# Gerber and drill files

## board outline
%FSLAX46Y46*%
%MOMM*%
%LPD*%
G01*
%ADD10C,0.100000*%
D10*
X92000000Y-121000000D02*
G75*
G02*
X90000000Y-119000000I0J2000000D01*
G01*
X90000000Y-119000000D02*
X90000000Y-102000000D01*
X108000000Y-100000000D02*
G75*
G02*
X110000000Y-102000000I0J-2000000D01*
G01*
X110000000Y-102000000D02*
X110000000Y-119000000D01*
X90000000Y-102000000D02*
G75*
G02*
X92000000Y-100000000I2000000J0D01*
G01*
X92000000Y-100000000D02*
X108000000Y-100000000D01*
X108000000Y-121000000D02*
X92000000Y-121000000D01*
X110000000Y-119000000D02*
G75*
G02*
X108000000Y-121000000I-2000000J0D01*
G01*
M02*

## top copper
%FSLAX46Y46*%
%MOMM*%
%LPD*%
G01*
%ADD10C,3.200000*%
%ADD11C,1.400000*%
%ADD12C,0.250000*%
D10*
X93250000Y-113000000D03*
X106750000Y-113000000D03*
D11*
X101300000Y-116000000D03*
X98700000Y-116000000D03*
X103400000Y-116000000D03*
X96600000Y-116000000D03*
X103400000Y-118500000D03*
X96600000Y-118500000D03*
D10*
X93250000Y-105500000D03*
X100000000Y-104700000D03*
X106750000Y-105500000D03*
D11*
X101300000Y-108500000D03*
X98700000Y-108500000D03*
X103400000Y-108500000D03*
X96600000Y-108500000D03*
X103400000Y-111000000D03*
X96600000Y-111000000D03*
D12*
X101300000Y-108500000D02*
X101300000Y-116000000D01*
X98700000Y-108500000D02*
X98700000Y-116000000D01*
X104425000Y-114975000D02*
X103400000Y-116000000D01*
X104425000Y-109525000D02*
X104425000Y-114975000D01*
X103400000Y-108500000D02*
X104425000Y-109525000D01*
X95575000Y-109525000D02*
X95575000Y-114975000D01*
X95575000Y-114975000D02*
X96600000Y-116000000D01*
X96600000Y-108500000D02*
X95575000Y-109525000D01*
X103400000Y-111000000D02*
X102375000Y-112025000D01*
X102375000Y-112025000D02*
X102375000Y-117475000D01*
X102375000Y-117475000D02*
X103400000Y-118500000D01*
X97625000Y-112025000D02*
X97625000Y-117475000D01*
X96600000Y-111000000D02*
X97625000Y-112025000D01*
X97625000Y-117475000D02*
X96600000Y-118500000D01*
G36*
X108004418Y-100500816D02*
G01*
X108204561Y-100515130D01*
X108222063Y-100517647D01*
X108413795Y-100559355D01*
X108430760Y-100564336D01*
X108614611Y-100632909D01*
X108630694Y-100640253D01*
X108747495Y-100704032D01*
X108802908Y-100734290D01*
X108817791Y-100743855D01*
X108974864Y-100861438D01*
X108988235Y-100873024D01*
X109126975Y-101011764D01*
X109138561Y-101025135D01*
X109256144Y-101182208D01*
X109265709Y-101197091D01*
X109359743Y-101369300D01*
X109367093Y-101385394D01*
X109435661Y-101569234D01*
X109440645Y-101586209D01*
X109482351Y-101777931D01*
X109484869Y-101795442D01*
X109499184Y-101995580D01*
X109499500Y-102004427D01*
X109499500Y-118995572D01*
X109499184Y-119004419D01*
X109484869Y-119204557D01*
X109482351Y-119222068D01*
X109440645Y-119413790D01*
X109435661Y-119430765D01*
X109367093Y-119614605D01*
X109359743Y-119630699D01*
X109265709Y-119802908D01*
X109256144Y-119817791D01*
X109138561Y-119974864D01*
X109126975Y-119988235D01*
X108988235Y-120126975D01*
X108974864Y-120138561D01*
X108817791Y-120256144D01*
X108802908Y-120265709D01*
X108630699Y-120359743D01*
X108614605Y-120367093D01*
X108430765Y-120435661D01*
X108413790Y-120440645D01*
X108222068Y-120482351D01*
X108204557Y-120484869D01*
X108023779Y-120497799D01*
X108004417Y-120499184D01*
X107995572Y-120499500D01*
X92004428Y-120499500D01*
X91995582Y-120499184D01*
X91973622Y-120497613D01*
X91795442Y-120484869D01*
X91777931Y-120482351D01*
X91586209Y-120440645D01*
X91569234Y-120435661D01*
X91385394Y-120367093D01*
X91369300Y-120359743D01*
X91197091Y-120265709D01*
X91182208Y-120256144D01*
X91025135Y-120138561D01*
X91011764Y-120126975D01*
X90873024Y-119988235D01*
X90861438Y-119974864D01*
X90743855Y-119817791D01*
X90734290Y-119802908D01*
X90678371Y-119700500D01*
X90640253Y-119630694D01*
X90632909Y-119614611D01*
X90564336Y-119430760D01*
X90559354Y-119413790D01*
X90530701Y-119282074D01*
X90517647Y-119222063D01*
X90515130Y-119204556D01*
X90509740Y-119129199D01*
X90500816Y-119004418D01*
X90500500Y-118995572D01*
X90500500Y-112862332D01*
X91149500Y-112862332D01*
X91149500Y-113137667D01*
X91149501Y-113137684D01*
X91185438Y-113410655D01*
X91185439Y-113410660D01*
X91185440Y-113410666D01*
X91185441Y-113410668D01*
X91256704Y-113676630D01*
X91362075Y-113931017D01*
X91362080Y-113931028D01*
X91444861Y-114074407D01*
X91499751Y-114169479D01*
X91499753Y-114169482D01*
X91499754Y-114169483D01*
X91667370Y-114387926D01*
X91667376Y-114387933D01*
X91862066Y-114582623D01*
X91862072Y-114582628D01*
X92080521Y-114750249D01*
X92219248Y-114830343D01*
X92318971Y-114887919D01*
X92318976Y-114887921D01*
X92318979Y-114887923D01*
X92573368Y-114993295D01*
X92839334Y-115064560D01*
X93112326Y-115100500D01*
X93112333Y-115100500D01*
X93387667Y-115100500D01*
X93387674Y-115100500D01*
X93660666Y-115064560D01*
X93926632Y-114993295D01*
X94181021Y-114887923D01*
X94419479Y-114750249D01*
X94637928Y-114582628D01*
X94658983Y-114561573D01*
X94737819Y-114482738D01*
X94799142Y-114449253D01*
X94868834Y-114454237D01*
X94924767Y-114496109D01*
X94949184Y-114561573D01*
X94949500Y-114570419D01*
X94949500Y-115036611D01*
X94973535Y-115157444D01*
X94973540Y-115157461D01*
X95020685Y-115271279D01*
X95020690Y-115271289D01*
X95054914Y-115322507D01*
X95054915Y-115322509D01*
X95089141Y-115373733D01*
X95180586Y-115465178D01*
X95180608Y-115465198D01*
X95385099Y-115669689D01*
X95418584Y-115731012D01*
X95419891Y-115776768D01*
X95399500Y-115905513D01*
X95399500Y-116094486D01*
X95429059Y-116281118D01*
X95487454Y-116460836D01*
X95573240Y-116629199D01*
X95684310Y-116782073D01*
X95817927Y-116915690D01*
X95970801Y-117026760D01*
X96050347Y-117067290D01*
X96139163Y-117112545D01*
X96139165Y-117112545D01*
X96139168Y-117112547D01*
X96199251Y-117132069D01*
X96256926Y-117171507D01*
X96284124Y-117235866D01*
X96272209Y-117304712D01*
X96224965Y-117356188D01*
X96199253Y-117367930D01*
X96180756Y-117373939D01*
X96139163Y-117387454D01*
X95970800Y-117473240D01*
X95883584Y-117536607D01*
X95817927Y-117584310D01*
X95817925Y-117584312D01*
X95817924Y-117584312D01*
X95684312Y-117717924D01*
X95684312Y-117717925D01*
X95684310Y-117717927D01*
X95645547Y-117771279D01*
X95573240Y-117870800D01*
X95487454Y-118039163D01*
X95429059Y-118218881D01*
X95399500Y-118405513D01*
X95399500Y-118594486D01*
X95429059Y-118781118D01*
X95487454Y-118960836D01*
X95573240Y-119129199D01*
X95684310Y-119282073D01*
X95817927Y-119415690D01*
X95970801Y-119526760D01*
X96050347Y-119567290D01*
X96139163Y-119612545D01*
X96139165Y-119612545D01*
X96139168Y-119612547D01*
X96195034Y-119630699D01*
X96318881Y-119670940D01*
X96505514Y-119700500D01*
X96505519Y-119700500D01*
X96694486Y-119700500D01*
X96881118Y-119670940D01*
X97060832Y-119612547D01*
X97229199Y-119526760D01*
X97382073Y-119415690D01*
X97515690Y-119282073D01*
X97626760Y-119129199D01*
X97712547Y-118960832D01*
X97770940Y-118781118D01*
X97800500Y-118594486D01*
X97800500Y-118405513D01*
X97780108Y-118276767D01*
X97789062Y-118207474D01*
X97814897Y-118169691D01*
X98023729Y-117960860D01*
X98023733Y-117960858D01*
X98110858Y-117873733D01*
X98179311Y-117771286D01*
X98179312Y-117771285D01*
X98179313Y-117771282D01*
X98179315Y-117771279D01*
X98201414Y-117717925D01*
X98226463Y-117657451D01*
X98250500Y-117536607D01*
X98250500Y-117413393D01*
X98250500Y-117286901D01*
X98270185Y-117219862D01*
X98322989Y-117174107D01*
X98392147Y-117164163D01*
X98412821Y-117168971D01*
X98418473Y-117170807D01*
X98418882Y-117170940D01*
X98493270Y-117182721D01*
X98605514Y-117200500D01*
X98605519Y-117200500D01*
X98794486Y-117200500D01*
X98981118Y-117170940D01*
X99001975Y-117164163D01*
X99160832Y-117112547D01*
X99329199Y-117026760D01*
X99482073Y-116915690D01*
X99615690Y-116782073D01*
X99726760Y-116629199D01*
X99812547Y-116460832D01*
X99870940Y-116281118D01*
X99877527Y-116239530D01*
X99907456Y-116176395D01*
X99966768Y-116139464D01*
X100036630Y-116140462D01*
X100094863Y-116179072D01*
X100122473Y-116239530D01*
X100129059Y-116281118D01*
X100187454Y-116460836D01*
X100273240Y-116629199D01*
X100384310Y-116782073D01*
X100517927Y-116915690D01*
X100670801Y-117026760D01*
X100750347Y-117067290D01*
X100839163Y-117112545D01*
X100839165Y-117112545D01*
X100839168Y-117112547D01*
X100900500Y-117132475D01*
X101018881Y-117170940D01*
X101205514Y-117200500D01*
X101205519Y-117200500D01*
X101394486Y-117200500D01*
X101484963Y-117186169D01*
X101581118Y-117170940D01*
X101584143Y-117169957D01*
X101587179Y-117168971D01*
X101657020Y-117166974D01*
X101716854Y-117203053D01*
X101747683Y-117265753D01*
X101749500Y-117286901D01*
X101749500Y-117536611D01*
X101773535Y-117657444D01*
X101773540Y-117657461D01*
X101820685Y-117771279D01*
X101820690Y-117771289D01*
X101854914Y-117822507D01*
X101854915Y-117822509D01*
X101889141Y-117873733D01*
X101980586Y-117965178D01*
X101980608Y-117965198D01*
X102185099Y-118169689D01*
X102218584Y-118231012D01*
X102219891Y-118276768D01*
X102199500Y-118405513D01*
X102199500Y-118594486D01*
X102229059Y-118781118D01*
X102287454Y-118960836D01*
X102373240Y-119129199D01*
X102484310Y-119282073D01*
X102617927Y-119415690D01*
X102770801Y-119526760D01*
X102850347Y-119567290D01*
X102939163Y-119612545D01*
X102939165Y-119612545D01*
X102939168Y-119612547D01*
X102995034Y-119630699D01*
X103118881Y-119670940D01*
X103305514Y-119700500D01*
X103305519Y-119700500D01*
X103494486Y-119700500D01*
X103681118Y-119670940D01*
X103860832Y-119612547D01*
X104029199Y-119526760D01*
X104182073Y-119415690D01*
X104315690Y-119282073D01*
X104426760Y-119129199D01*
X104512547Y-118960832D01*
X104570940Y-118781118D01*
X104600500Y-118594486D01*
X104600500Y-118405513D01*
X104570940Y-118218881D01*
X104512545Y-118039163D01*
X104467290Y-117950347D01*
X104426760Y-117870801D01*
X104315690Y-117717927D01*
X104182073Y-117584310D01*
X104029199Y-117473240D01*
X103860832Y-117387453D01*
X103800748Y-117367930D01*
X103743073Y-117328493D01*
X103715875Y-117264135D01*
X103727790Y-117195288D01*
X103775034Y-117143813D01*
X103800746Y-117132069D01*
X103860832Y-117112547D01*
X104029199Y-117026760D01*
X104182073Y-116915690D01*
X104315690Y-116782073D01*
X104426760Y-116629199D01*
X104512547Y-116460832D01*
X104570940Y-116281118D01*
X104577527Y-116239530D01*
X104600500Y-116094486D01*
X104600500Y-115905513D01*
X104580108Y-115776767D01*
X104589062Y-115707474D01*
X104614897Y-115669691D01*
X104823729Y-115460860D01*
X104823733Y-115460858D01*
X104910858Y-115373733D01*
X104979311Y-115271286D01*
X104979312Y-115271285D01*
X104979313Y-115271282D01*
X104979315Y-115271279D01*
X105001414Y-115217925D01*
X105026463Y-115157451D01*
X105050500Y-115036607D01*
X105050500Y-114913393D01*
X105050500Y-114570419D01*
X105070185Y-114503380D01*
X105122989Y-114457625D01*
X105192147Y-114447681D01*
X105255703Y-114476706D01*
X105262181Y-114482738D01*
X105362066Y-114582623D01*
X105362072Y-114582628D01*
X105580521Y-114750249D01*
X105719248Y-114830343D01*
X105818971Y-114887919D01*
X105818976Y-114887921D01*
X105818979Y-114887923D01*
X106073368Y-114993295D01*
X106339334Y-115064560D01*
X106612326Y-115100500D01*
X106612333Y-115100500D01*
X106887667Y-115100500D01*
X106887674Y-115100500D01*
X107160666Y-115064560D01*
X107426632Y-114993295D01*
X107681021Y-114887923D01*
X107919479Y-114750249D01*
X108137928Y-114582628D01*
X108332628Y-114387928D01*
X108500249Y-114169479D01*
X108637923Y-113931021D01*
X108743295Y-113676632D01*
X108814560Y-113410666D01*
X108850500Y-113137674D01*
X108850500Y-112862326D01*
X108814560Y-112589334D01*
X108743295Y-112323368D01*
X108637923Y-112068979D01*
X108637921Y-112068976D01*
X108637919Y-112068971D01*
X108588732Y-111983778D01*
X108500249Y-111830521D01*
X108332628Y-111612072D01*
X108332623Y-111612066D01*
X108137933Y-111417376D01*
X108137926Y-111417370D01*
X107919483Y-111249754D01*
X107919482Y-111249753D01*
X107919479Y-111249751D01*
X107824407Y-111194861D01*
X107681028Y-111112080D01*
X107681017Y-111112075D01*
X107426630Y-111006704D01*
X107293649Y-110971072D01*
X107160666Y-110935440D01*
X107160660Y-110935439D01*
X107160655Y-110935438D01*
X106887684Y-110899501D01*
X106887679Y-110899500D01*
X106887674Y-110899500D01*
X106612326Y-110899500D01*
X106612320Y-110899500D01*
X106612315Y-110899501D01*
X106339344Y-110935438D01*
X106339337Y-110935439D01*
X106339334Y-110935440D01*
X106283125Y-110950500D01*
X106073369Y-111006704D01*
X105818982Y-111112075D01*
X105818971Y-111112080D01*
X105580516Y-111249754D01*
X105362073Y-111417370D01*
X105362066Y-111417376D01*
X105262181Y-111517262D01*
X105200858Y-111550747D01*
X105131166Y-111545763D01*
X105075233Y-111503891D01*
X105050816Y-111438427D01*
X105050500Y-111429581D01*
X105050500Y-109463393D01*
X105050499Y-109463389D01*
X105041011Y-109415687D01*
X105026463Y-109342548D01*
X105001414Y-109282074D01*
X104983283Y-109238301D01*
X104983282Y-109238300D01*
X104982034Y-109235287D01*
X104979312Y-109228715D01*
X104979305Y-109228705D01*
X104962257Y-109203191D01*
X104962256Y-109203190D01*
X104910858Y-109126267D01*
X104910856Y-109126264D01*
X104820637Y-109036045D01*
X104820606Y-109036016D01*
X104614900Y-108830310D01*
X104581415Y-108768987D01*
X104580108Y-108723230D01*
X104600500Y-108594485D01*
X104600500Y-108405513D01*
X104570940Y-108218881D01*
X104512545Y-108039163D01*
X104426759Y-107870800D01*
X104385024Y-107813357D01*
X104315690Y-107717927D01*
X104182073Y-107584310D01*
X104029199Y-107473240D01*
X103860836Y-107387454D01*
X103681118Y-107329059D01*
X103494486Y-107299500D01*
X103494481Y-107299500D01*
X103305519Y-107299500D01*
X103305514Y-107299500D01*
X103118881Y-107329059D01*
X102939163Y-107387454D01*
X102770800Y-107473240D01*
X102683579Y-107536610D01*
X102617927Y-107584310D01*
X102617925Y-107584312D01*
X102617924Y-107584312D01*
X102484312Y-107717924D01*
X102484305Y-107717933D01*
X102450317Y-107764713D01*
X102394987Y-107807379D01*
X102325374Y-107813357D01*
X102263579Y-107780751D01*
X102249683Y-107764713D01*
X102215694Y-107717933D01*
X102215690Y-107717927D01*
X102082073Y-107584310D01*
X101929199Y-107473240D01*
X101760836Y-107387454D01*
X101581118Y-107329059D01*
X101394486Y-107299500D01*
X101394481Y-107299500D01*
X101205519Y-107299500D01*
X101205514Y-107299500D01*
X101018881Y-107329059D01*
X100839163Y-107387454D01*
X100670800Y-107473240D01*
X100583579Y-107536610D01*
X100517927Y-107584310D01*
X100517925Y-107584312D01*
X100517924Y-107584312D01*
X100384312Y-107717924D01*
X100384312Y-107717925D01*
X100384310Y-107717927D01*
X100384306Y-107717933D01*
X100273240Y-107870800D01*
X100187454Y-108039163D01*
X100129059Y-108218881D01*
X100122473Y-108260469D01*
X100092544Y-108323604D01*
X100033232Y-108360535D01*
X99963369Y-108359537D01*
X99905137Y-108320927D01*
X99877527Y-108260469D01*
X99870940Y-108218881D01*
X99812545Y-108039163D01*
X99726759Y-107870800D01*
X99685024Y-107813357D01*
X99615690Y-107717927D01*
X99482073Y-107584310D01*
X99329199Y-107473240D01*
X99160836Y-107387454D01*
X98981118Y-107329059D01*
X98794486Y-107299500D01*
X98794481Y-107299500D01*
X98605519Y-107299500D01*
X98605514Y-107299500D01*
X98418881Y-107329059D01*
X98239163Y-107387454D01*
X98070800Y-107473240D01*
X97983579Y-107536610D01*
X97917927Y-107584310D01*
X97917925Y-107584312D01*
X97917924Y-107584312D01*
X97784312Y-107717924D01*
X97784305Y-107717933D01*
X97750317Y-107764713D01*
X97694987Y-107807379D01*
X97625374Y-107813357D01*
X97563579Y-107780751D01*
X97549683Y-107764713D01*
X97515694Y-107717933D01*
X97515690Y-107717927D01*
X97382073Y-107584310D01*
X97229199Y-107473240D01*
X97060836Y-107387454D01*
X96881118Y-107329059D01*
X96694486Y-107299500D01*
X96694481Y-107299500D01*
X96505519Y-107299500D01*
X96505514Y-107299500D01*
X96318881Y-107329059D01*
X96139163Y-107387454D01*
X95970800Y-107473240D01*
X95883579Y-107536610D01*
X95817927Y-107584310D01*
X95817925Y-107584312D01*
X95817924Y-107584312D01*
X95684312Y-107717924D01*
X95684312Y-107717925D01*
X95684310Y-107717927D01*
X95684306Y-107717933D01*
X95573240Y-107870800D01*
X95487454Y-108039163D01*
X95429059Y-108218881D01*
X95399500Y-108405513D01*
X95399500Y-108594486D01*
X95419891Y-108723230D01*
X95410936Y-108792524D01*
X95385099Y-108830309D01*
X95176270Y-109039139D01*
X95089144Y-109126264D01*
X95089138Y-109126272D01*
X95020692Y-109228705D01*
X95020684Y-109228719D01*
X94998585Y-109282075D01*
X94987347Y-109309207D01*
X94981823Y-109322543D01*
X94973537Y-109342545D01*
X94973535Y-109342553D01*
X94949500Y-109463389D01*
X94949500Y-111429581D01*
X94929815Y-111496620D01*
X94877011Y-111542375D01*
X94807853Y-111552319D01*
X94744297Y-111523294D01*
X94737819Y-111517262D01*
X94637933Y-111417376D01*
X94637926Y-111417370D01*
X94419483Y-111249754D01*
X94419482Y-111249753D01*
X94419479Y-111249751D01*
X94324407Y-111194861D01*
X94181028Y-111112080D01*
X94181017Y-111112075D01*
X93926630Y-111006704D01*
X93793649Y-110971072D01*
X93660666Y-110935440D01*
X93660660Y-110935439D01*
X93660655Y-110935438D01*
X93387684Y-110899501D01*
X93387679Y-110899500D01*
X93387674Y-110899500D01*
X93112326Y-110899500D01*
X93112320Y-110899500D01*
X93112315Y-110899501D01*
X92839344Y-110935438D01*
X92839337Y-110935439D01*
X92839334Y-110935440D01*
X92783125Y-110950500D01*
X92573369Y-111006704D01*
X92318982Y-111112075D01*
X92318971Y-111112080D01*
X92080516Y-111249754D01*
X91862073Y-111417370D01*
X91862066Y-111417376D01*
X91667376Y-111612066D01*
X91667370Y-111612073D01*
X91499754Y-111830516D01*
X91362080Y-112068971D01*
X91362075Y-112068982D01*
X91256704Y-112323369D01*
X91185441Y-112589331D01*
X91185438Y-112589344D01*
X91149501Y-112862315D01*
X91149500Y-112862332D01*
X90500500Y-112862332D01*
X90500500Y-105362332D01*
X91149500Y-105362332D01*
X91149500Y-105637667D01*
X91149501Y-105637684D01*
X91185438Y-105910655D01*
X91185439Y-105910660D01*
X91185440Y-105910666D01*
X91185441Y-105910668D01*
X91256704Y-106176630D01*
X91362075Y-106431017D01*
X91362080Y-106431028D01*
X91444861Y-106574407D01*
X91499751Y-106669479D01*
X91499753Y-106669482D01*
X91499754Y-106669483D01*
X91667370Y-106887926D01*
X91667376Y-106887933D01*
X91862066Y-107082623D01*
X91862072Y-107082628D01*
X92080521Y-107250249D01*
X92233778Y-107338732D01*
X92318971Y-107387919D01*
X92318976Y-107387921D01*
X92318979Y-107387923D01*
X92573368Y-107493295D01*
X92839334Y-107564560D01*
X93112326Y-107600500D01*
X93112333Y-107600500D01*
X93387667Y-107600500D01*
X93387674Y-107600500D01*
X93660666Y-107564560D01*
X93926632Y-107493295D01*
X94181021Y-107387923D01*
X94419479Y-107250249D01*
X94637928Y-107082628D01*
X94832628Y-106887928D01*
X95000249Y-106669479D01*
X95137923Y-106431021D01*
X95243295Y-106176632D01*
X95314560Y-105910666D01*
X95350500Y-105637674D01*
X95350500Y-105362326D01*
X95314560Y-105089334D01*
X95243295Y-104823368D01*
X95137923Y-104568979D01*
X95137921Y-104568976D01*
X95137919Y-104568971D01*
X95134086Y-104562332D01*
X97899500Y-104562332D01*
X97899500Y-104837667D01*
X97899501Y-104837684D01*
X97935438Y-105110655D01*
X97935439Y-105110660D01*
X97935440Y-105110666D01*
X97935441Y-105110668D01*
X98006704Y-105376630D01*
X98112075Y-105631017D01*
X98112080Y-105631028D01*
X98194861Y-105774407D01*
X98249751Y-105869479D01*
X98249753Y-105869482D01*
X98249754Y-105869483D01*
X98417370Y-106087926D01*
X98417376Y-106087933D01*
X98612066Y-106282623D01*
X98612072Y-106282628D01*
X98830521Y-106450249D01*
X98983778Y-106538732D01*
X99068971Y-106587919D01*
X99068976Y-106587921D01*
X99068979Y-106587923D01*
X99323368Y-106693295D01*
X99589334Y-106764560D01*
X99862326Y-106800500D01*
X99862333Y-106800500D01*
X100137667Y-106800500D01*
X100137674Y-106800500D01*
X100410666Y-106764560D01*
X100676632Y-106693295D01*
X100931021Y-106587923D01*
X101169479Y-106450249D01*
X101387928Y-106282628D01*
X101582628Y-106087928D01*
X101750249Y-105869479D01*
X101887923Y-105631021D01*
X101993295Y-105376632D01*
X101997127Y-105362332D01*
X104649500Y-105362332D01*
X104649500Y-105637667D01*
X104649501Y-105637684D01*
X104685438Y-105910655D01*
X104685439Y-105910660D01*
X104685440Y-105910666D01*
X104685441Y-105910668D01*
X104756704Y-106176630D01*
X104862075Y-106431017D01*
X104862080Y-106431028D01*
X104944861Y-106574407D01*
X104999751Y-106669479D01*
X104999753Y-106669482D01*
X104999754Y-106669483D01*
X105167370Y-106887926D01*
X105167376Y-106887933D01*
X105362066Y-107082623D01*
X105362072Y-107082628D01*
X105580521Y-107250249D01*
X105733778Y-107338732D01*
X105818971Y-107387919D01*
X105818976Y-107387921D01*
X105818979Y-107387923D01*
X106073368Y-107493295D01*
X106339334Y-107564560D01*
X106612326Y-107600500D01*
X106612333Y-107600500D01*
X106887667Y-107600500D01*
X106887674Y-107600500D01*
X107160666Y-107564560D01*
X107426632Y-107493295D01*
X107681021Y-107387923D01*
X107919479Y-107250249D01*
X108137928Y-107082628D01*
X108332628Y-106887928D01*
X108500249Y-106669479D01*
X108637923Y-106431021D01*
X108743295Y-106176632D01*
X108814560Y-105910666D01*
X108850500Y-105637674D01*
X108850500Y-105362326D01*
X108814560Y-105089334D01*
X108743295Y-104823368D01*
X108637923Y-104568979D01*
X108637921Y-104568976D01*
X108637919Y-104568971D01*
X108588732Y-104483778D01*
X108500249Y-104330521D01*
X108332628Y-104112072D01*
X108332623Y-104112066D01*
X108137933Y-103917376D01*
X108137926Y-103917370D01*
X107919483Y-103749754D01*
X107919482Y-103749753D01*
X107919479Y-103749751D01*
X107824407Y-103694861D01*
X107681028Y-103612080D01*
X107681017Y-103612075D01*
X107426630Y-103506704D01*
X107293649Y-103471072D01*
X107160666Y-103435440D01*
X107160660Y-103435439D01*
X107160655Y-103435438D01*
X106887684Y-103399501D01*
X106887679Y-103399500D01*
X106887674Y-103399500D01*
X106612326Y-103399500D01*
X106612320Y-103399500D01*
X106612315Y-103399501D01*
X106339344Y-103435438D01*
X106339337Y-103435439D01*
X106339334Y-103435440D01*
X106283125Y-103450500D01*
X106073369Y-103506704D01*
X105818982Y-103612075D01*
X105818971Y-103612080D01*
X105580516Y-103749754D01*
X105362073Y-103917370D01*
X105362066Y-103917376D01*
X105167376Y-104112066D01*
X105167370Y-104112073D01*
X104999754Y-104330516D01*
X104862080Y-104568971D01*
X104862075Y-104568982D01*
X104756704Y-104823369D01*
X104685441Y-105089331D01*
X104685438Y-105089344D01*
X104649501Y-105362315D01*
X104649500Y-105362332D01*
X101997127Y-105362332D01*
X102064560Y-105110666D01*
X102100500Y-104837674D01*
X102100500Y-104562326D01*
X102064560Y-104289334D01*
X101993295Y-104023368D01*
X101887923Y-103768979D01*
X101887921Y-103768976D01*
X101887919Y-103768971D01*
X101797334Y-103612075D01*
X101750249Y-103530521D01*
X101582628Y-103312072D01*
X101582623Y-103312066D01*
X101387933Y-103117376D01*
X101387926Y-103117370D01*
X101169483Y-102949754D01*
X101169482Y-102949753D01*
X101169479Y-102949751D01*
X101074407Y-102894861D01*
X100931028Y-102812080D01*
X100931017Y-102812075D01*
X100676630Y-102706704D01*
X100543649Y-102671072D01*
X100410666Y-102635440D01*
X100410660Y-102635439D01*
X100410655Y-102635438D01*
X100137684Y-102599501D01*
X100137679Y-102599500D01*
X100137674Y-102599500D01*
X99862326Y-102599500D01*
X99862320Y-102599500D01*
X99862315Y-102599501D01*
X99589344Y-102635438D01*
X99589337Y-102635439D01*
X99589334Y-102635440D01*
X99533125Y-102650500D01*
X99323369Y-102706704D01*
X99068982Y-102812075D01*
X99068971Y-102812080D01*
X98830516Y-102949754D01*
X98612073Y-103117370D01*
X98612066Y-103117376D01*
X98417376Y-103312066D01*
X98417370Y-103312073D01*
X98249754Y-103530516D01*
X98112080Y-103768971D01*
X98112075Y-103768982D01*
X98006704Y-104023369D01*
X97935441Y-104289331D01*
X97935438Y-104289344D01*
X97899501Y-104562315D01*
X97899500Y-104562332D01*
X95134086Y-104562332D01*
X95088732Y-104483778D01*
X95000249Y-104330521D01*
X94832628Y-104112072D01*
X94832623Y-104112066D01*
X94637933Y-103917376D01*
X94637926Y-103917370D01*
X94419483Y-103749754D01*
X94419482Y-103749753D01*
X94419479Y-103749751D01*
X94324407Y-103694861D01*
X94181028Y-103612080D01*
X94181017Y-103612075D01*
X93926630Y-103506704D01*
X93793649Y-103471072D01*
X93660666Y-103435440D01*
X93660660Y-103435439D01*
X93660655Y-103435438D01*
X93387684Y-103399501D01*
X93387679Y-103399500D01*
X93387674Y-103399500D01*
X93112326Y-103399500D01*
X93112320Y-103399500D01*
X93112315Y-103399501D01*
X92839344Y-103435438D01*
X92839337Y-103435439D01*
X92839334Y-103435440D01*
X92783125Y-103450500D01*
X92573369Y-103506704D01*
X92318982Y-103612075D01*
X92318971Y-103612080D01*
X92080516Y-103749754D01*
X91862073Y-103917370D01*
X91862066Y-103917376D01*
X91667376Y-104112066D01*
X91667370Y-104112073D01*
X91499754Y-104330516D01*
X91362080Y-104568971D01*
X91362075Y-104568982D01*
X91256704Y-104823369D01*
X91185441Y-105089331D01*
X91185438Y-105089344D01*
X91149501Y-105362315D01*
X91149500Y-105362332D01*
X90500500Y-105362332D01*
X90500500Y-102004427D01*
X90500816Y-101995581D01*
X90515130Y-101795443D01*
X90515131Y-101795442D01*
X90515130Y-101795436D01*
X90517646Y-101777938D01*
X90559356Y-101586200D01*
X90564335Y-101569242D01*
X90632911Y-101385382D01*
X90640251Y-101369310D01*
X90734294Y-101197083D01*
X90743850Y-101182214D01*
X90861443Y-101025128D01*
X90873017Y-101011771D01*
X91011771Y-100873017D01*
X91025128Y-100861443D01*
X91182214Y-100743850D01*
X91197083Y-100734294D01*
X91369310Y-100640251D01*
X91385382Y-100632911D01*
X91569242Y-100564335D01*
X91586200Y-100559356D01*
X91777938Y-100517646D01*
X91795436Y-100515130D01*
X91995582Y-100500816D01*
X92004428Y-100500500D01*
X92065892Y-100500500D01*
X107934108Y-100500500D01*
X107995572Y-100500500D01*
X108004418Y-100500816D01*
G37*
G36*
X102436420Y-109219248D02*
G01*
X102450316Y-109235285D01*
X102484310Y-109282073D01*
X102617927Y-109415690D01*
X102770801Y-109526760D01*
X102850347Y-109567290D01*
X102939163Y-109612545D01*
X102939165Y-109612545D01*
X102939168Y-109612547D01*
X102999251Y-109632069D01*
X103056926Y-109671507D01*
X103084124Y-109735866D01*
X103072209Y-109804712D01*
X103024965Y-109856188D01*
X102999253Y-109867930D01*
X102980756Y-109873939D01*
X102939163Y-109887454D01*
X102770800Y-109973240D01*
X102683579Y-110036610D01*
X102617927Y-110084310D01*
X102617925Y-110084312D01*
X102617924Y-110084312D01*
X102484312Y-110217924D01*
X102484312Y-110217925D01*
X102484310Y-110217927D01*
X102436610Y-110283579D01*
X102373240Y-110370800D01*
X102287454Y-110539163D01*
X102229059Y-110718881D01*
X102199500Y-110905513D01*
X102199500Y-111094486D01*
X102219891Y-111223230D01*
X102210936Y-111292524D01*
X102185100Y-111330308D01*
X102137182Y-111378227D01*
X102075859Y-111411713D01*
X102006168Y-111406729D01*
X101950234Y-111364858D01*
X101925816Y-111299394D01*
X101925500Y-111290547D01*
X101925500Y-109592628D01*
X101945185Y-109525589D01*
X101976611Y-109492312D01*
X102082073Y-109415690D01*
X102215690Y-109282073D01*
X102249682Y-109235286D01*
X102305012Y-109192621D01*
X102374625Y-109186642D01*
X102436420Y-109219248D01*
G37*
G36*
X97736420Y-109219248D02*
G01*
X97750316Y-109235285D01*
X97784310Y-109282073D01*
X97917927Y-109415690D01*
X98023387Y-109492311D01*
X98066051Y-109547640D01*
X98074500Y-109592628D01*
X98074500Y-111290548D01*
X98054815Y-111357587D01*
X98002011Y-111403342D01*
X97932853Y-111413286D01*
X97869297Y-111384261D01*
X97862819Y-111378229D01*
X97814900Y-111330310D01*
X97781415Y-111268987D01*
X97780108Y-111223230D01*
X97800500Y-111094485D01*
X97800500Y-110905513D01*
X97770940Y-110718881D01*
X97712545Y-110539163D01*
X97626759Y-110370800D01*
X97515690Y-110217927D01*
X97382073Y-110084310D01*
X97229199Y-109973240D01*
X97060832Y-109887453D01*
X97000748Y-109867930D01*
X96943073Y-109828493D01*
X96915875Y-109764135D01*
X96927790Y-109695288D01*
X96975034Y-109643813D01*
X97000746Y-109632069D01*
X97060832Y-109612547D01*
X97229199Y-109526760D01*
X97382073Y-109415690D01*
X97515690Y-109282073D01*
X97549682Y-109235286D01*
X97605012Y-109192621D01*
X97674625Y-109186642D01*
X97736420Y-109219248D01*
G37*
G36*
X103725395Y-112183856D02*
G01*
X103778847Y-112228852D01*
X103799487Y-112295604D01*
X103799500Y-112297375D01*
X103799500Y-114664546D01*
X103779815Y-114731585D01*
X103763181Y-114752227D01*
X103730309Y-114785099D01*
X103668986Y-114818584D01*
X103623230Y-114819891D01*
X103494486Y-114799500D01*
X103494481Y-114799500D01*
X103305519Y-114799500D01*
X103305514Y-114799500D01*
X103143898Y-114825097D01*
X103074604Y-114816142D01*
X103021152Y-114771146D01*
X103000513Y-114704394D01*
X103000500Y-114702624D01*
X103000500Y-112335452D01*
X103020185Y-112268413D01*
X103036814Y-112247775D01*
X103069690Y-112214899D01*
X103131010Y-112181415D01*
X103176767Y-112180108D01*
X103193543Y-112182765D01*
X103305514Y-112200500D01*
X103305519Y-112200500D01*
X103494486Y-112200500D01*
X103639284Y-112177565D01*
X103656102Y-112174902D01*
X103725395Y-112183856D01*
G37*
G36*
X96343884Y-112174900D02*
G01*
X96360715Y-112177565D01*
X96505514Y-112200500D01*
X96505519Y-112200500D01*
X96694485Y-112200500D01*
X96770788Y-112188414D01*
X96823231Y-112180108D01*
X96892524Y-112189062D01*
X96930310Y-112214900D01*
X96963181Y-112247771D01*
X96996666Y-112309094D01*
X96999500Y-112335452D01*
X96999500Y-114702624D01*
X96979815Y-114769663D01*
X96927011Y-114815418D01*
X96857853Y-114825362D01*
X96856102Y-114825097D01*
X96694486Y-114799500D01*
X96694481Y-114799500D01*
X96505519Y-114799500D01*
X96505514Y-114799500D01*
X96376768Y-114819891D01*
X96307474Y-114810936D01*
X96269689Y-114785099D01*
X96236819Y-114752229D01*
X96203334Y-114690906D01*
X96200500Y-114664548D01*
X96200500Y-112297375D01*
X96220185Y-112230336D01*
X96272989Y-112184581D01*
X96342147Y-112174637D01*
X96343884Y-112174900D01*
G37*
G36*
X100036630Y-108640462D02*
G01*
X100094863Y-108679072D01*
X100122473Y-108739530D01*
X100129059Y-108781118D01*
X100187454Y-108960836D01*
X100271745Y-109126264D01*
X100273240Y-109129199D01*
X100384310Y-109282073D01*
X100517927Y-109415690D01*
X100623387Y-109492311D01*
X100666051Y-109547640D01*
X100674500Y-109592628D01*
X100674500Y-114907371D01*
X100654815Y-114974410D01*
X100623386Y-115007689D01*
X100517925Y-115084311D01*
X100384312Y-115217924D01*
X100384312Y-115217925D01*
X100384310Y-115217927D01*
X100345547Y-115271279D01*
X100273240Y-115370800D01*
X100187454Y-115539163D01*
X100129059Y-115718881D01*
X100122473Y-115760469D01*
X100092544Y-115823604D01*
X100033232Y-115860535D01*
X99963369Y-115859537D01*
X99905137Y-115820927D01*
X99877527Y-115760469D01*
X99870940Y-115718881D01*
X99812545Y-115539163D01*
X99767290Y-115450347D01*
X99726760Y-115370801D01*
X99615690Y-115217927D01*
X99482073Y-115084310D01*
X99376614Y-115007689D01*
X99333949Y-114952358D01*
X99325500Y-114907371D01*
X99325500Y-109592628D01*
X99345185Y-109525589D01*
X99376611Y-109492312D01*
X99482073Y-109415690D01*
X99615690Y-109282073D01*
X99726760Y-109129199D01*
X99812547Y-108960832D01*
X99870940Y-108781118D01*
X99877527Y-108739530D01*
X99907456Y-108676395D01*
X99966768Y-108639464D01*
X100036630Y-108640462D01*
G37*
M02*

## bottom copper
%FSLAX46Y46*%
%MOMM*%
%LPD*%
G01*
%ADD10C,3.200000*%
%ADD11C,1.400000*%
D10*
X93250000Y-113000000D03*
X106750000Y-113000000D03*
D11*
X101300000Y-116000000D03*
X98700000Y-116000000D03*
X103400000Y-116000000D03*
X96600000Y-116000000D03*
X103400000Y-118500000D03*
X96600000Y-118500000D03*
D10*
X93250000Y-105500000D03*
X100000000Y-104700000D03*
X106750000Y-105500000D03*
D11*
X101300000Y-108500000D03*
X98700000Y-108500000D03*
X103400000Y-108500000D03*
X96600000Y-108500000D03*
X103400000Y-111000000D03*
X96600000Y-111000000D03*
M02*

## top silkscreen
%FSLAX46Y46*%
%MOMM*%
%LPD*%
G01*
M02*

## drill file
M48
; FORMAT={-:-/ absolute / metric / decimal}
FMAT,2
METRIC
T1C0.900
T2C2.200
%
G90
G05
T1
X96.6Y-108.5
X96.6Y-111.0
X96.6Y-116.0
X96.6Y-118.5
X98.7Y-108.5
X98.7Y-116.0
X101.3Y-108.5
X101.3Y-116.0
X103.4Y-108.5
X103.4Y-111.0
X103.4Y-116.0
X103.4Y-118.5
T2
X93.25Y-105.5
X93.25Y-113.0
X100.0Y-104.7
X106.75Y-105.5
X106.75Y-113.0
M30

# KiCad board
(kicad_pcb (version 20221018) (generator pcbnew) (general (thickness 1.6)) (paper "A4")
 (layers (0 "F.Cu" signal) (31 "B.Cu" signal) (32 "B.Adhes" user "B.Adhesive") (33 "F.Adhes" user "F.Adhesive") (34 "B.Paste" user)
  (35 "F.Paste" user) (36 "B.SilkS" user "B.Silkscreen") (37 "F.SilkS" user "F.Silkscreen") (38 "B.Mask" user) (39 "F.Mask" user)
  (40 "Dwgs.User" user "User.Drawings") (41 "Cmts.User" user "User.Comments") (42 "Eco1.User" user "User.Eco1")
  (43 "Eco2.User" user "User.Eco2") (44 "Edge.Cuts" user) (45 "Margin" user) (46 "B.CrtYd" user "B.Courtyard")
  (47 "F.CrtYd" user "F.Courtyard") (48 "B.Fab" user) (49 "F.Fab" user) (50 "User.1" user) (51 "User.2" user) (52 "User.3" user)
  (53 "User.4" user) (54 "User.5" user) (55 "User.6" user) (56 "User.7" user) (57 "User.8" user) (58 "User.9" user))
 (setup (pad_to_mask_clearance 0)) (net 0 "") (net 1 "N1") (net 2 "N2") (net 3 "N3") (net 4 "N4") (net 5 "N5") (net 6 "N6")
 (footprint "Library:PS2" (layer "F.Cu") (at 100 107.5)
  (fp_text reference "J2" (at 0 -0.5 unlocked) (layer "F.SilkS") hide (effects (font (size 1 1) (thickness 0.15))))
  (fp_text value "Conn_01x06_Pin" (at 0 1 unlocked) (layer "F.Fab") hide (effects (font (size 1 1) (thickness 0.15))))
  (pad "" thru_hole circle (at -6.75 5.5) (size 3.2 3.2) (drill 2.2) (layers "*.Cu" "*.Mask"))
  (pad "" thru_hole circle (at 6.75 5.5 90) (size 3.2 3.2) (drill 2.2) (layers "*.Cu" "*.Mask"))
  (pad "1" thru_hole circle (at 1.3 8.5) (size 1.4 1.4) (drill 0.9) (layers "*.Cu" "*.Mask") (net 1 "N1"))
  (pad "2" thru_hole circle (at -1.3 8.5) (size 1.4 1.4) (drill 0.9) (layers "*.Cu" "*.Mask") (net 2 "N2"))
  (pad "3" thru_hole circle (at 3.4 8.5) (size 1.4 1.4) (drill 0.9) (layers "*.Cu" "*.Mask") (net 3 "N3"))
  (pad "4" thru_hole circle (at -3.4 8.5) (size 1.4 1.4) (drill 0.9) (layers "*.Cu" "*.Mask") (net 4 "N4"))
  (pad "5" thru_hole circle (at 3.4 11) (size 1.4 1.4) (drill 0.9) (layers "*.Cu" "*.Mask") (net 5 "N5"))
  (pad "6" thru_hole circle (at -3.4 11) (size 1.4 1.4) (drill 0.9) (layers "*.Cu" "*.Mask") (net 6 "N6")))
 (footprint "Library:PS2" (layer "F.Cu") (at 100 100)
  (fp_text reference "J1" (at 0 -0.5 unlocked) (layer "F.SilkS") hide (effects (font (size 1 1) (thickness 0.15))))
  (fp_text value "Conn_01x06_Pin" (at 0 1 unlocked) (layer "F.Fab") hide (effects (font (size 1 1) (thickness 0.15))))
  (pad "" thru_hole circle (at -6.75 5.5) (size 3.2 3.2) (drill 2.2) (layers "*.Cu" "*.Mask"))
  (pad "" thru_hole circle (at 0 4.7) (size 3.2 3.2) (drill 2.2) (layers "*.Cu" "*.Mask"))
  (pad "" thru_hole circle (at 6.75 5.5 90) (size 3.2 3.2) (drill 2.2) (layers "*.Cu" "*.Mask"))
  (pad "1" thru_hole circle (at 1.3 8.5) (size 1.4 1.4) (drill 0.9) (layers "*.Cu" "*.Mask") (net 1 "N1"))
  (pad "2" thru_hole circle (at -1.3 8.5) (size 1.4 1.4) (drill 0.9) (layers "*.Cu" "*.Mask") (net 2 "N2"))
  (pad "3" thru_hole circle (at 3.4 8.5) (size 1.4 1.4) (drill 0.9) (layers "*.Cu" "*.Mask") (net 3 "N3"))
  (pad "4" thru_hole circle (at -3.4 8.5) (size 1.4 1.4) (drill 0.9) (layers "*.Cu" "*.Mask") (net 4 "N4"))
  (pad "5" thru_hole circle (at 3.4 11) (size 1.4 1.4) (drill 0.9) (layers "*.Cu" "*.Mask") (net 5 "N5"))
  (pad "6" thru_hole circle (at -3.4 11) (size 1.4 1.4) (drill 0.9) (layers "*.Cu" "*.Mask") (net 6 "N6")))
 (gr_arc (start 92 121) (mid 90.585786 120.414214) (end 90 119) (stroke (width 0.1) (type default)) (layer "Edge.Cuts"))
 (gr_line (start 90 119) (end 90 102) (stroke (width 0.1) (type default)) (layer "Edge.Cuts"))
 (gr_arc (start 108 100) (mid 109.414214 100.585786) (end 110 102) (stroke (width 0.1) (type default)) (layer "Edge.Cuts"))
 (gr_line (start 110 102) (end 110 119) (stroke (width 0.1) (type default)) (layer "Edge.Cuts"))
 (gr_arc (start 90 102) (mid 90.585786 100.585786) (end 92 100) (stroke (width 0.1) (type default)) (layer "Edge.Cuts"))
 (gr_line (start 92 100) (end 108 100) (stroke (width 0.1) (type default)) (layer "Edge.Cuts"))
 (gr_line (start 108 121) (end 92 121) (stroke (width 0.1) (type default)) (layer "Edge.Cuts"))
 (gr_arc (start 110 119) (mid 109.414214 120.414214) (end 108 121) (stroke (width 0.1) (type default)) (layer "Edge.Cuts"))
 (segment (start 101.3 108.5) (end 101.3 116) (width 0.25) (layer "F.Cu") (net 1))
 (segment (start 98.7 108.5) (end 98.7 116) (width 0.25) (layer "F.Cu") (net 2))
 (segment (start 104.425 114.975) (end 103.4 116) (width 0.25) (layer "F.Cu") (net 3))
 (segment (start 104.425 109.525) (end 104.425 114.975) (width 0.25) (layer "F.Cu") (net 3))
 (segment (start 103.4 108.5) (end 104.425 109.525) (width 0.25) (layer "F.Cu") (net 3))
 (segment (start 95.575 109.525) (end 95.575 114.975) (width 0.25) (layer "F.Cu") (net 4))
 (segment (start 95.575 114.975) (end 96.6 116) (width 0.25) (layer "F.Cu") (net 4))
 (segment (start 96.6 108.5) (end 95.575 109.525) (width 0.25) (layer "F.Cu") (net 4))
 (segment (start 103.4 111) (end 102.375 112.025) (width 0.25) (layer "F.Cu") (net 5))
 (segment (start 102.375 112.025) (end 102.375 117.475) (width 0.25) (layer "F.Cu") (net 5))
 (segment (start 102.375 117.475) (end 103.4 118.5) (width 0.25) (layer "F.Cu") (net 5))
 (segment (start 97.625 112.025) (end 97.625 117.475) (width 0.25) (layer "F.Cu") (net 6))
 (segment (start 96.6 111) (end 97.625 112.025) (width 0.25) (layer "F.Cu") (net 6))
 (segment (start 97.625 117.475) (end 96.6 118.5) (width 0.25) (layer "F.Cu") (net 6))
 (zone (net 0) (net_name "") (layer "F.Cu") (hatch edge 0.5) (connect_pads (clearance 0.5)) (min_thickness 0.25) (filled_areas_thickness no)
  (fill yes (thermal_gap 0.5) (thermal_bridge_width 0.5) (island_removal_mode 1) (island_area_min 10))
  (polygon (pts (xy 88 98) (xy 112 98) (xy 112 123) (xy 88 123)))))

